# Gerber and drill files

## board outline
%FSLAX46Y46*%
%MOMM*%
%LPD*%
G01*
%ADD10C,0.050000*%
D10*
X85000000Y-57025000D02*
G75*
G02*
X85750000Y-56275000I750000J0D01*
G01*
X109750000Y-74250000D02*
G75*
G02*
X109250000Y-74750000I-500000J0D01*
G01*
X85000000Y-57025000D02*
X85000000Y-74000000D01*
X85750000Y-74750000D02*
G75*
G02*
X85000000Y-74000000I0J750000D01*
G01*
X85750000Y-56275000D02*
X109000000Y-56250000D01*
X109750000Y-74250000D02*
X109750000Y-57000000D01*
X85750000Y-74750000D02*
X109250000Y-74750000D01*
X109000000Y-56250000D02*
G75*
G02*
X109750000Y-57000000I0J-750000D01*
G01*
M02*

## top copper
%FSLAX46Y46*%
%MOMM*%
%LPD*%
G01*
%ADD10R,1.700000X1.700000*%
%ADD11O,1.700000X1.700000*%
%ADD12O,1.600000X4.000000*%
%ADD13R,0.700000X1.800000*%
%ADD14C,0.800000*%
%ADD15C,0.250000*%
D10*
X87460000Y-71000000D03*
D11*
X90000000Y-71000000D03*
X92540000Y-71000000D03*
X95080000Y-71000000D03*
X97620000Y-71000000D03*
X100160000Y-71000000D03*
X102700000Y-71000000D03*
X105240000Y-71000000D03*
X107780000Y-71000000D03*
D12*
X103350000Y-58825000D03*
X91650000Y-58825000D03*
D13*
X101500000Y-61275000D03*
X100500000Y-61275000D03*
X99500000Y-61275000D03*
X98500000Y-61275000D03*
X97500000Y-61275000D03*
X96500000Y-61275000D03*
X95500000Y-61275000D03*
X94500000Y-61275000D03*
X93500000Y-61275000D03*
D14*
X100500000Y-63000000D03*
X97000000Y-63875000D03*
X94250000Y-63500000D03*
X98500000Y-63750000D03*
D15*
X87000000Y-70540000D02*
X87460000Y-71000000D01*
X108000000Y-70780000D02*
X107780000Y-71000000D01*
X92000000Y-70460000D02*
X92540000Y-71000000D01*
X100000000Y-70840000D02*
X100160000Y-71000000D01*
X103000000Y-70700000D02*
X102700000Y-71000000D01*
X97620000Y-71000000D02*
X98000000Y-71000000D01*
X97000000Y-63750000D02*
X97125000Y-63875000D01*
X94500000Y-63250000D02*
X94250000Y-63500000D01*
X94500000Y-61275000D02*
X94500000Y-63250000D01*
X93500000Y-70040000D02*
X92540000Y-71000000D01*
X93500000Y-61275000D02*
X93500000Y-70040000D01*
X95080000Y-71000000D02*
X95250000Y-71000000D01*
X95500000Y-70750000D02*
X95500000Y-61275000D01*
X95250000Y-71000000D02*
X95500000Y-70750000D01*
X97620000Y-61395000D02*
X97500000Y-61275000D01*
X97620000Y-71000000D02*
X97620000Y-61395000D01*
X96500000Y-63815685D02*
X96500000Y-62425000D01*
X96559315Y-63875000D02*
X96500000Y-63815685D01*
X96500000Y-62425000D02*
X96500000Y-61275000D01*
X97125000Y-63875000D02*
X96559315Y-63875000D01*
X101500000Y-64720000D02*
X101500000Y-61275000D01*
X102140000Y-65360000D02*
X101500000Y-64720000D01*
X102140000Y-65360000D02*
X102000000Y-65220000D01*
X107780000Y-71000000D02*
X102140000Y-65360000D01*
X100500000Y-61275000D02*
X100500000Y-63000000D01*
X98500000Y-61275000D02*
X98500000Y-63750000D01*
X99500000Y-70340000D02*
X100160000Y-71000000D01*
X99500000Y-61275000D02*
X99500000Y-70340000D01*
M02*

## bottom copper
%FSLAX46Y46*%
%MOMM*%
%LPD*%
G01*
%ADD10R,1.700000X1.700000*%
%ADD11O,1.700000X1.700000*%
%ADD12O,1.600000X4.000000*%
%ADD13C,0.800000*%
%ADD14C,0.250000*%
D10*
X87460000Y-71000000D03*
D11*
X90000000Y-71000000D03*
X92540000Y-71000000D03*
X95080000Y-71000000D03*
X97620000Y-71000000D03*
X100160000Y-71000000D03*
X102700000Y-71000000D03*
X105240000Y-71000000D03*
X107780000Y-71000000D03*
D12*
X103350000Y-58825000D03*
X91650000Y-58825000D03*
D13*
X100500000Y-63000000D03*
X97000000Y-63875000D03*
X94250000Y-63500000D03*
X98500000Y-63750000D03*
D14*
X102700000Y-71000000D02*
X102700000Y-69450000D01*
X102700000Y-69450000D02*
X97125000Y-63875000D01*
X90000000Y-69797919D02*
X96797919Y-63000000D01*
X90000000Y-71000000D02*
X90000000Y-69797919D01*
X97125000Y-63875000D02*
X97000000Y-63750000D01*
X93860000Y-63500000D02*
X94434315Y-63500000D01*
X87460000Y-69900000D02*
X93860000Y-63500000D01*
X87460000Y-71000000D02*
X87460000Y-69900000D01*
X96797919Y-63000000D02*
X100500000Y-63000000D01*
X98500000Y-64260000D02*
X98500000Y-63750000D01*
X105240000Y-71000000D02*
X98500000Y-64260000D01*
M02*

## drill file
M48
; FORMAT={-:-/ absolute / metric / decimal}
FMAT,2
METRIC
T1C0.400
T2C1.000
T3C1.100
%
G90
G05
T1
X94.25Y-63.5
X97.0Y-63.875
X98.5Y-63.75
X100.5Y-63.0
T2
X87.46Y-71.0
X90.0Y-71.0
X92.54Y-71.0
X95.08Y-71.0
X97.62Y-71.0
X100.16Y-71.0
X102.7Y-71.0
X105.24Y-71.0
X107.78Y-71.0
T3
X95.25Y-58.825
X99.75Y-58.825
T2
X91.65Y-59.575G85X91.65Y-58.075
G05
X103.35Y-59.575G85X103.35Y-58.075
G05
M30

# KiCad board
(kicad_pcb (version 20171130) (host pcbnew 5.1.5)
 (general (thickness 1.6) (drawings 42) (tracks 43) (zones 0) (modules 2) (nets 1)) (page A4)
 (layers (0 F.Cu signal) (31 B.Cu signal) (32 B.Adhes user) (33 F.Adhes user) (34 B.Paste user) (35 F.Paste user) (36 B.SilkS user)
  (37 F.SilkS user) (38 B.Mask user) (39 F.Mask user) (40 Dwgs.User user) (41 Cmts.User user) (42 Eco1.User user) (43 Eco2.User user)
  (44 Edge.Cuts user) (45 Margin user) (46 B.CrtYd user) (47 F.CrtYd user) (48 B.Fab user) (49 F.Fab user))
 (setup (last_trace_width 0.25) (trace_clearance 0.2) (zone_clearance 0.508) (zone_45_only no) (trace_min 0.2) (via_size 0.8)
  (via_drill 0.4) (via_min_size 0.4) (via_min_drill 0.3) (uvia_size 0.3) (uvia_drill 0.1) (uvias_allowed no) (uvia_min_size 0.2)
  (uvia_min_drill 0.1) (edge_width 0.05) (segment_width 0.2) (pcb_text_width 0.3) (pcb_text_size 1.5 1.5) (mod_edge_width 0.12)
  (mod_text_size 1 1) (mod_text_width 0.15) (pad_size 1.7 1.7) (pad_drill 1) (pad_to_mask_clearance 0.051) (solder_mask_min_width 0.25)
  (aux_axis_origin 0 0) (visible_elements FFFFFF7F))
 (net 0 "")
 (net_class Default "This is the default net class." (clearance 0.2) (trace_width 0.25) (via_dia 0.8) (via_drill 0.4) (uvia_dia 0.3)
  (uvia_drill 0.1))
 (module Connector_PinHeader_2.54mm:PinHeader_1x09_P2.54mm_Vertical (layer F.Cu) (at 87.46 71 90)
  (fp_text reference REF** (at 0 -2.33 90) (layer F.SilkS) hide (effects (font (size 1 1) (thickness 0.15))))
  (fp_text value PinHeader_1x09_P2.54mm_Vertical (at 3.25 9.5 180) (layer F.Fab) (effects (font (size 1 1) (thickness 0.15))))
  (pad 1 thru_hole rect (at 0 0 90) (size 1.7 1.7) (drill 1) (layers *.Cu *.Mask))
  (pad 4 thru_hole oval (at 0 2.54 90) (size 1.7 1.7) (drill 1) (layers *.Cu *.Mask))
  (pad 9 thru_hole oval (at 0 5.08 90) (size 1.7 1.7) (drill 1) (layers *.Cu *.Mask))
  (pad 8 thru_hole oval (at 0 7.62 90) (size 1.7 1.7) (drill 1) (layers *.Cu *.Mask))
  (pad 7 thru_hole oval (at 0 10.16 90) (size 1.7 1.7) (drill 1) (layers *.Cu *.Mask))
  (pad 6 thru_hole oval (at 0 12.7 90) (size 1.7 1.7) (drill 1) (layers *.Cu *.Mask))
  (pad 2 thru_hole oval (at 0 15.24 90) (size 1.7 1.7) (drill 1) (layers *.Cu *.Mask))
  (pad 3 thru_hole oval (at 0 17.78 90) (size 1.7 1.7) (drill 1) (layers *.Cu *.Mask))
  (pad 5 thru_hole oval (at 0 20.32 90) (size 1.7 1.7) (drill 1) (layers *.Cu *.Mask)))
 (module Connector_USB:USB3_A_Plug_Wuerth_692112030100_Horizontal (layer F.Cu) (at 97.5 59.5 90)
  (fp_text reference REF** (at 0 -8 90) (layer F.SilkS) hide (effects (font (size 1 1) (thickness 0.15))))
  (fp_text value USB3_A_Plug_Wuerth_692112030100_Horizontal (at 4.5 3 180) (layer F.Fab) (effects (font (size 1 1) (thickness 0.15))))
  (pad 10 thru_hole oval (at 0.675 5.85 180) (size 1.6 4) (drill oval 1 2.5) (layers *.Cu *.Mask))
  (pad 10 thru_hole oval (at 0.675 -5.85 180) (size 1.6 4) (drill oval 1 2.5) (layers *.Cu *.Mask))
  (pad 5 smd rect (at -1.775 4 180) (size 0.7 1.8) (layers F.Cu F.Paste F.Mask))
  (pad 4 smd rect (at -1.775 3 180) (size 0.7 1.8) (layers F.Cu F.Paste F.Mask))
  (pad 6 smd rect (at -1.775 2 180) (size 0.7 1.8) (layers F.Cu F.Paste F.Mask))
  (pad 3 smd rect (at -1.775 1 180) (size 0.7 1.8) (layers F.Cu F.Paste F.Mask))
  (pad 7 smd rect (at -1.775 0 180) (size 0.7 1.8) (layers F.Cu F.Paste F.Mask))
  (pad 2 smd rect (at -1.775 -1 180) (size 0.7 1.8) (layers F.Cu F.Paste F.Mask))
  (pad 8 smd rect (at -1.775 -2 180) (size 0.7 1.8) (layers F.Cu F.Paste F.Mask))
  (pad 1 smd rect (at -1.775 -3 180) (size 0.7 1.8) (layers F.Cu F.Paste F.Mask))
  (pad 9 smd rect (at -1.775 -4 90) (size 1.8 0.7) (layers F.Cu F.Paste F.Mask))
  (pad "" np_thru_hole circle (at 0.675 2.25 180) (size 1.1 1.1) (drill 1.1) (layers *.Cu *.Mask))
  (pad "" np_thru_hole circle (at 0.675 -2.25 180) (size 1.1 1.1) (drill 1.1) (layers *.Cu *.Mask)))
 (gr_arc (start 85.75 57.025) (end 85.75 56.275) (angle -90) (layer Edge.Cuts) (width 0.05))
 (gr_arc (start 109.25 74.25) (end 109.25 74.75) (angle -90) (layer Edge.Cuts) (width 0.05))
 (gr_line (start 85 57.025) (end 85 74) (layer Edge.Cuts) (width 0.05))
 (gr_arc (start 85.75 74) (end 85 74) (angle -90) (layer Edge.Cuts) (width 0.05))
 (gr_line (start 85.75 56.275) (end 109 56.25) (layer Edge.Cuts) (width 0.05))
 (gr_line (start 109.75 74.25) (end 109.75 57) (layer Edge.Cuts) (width 0.05))
 (gr_line (start 85.75 74.75) (end 109.25 74.75) (layer Edge.Cuts) (width 0.05))
 (gr_arc (start 109 57) (end 109.75 57) (angle -90) (layer Edge.Cuts) (width 0.05))
 (segment (start 87 70.54) (end 87.46 71) (width 0.25) (layer F.Cu) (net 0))
 (segment (start 108 70.78) (end 107.78 71) (width 0.25) (layer F.Cu) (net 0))
 (segment (start 92 70.46) (end 92.54 71) (width 0.25) (layer F.Cu) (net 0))
 (segment (start 100 70.84) (end 100.16 71) (width 0.25) (layer F.Cu) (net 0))
 (segment (start 103 70.7) (end 102.7 71) (width 0.25) (layer F.Cu) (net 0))
 (segment (start 97.62 71) (end 98 71) (width 0.25) (layer F.Cu) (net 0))
 (segment (start 102.7 71) (end 102.7 69.45) (width 0.25) (layer B.Cu) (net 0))
 (segment (start 102.7 69.45) (end 97.125 63.875) (width 0.25) (layer B.Cu) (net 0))
 (segment (start 90 69.797919) (end 96.797919 63) (width 0.25) (layer B.Cu) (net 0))
 (segment (start 90 71) (end 90 69.797919) (width 0.25) (layer B.Cu) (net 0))
 (via (at 100.5 63) (size 0.8) (drill 0.4) (layers F.Cu B.Cu) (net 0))
 (segment (start 97.125 63.875) (end 97 63.75) (width 0.25) (layer B.Cu) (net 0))
 (via (at 97 63.875) (size 0.8) (drill 0.4) (layers F.Cu B.Cu) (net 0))
 (via (at 94.25 63.5) (size 0.8) (drill 0.4) (layers F.Cu B.Cu) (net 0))
 (segment (start 97 63.75) (end 97.125 63.875) (width 0.25) (layer F.Cu) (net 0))
 (segment (start 93.86 63.5) (end 94.434315 63.5) (width 0.25) (layer B.Cu) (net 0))
 (segment (start 87.46 69.9) (end 93.86 63.5) (width 0.25) (layer B.Cu) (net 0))
 (segment (start 87.46 71) (end 87.46 69.9) (width 0.25) (layer B.Cu) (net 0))
 (segment (start 94.5 63.25) (end 94.25 63.5) (width 0.25) (layer F.Cu) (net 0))
 (segment (start 94.5 61.275) (end 94.5 63.25) (width 0.25) (layer F.Cu) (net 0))
 (segment (start 93.5 70.04) (end 92.54 71) (width 0.25) (layer F.Cu) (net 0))
 (segment (start 93.5 61.275) (end 93.5 70.04) (width 0.25) (layer F.Cu) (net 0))
 (segment (start 95.08 71) (end 95.25 71) (width 0.25) (layer F.Cu) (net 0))
 (segment (start 95.5 70.75) (end 95.5 61.275) (width 0.25) (layer F.Cu) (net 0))
 (segment (start 95.25 71) (end 95.5 70.75) (width 0.25) (layer F.Cu) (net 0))
 (segment (start 97.62 61.395) (end 97.5 61.275) (width 0.25) (layer F.Cu) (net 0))
 (segment (start 97.62 71) (end 97.62 61.395) (width 0.25) (layer F.Cu) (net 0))
 (segment (start 96.5 63.815685) (end 96.5 62.425) (width 0.25) (layer F.Cu) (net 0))
 (segment (start 96.559315 63.875) (end 96.5 63.815685) (width 0.25) (layer F.Cu) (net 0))
 (segment (start 96.5 62.425) (end 96.5 61.275) (width 0.25) (layer F.Cu) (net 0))
 (segment (start 97.125 63.875) (end 96.559315 63.875) (width 0.25) (layer F.Cu) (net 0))
 (segment (start 101.5 64.72) (end 101.5 61.275) (width 0.25) (layer F.Cu) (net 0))
 (segment (start 102.14 65.36) (end 101.5 64.72) (width 0.25) (layer F.Cu) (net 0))
 (segment (start 102.14 65.36) (end 102 65.22) (width 0.25) (layer F.Cu) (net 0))
 (segment (start 107.78 71) (end 102.14 65.36) (width 0.25) (layer F.Cu) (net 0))
 (segment (start 100.5 61.275) (end 100.5 63) (width 0.25) (layer F.Cu) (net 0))
 (segment (start 96.797919 63) (end 100.5 63) (width 0.25) (layer B.Cu) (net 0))
 (segment (start 98.5 61.275) (end 98.5 63.75) (width 0.25) (layer F.Cu) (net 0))
 (via (at 98.5 63.75) (size 0.8) (drill 0.4) (layers F.Cu B.Cu) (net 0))
 (segment (start 98.5 64.26) (end 98.5 63.75) (width 0.25) (layer B.Cu) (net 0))
 (segment (start 105.24 71) (end 98.5 64.26) (width 0.25) (layer B.Cu) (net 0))
 (segment (start 99.5 70.34) (end 100.16 71) (width 0.25) (layer F.Cu) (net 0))
 (segment (start 99.5 61.275) (end 99.5 70.34) (width 0.25) (layer F.Cu) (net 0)))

